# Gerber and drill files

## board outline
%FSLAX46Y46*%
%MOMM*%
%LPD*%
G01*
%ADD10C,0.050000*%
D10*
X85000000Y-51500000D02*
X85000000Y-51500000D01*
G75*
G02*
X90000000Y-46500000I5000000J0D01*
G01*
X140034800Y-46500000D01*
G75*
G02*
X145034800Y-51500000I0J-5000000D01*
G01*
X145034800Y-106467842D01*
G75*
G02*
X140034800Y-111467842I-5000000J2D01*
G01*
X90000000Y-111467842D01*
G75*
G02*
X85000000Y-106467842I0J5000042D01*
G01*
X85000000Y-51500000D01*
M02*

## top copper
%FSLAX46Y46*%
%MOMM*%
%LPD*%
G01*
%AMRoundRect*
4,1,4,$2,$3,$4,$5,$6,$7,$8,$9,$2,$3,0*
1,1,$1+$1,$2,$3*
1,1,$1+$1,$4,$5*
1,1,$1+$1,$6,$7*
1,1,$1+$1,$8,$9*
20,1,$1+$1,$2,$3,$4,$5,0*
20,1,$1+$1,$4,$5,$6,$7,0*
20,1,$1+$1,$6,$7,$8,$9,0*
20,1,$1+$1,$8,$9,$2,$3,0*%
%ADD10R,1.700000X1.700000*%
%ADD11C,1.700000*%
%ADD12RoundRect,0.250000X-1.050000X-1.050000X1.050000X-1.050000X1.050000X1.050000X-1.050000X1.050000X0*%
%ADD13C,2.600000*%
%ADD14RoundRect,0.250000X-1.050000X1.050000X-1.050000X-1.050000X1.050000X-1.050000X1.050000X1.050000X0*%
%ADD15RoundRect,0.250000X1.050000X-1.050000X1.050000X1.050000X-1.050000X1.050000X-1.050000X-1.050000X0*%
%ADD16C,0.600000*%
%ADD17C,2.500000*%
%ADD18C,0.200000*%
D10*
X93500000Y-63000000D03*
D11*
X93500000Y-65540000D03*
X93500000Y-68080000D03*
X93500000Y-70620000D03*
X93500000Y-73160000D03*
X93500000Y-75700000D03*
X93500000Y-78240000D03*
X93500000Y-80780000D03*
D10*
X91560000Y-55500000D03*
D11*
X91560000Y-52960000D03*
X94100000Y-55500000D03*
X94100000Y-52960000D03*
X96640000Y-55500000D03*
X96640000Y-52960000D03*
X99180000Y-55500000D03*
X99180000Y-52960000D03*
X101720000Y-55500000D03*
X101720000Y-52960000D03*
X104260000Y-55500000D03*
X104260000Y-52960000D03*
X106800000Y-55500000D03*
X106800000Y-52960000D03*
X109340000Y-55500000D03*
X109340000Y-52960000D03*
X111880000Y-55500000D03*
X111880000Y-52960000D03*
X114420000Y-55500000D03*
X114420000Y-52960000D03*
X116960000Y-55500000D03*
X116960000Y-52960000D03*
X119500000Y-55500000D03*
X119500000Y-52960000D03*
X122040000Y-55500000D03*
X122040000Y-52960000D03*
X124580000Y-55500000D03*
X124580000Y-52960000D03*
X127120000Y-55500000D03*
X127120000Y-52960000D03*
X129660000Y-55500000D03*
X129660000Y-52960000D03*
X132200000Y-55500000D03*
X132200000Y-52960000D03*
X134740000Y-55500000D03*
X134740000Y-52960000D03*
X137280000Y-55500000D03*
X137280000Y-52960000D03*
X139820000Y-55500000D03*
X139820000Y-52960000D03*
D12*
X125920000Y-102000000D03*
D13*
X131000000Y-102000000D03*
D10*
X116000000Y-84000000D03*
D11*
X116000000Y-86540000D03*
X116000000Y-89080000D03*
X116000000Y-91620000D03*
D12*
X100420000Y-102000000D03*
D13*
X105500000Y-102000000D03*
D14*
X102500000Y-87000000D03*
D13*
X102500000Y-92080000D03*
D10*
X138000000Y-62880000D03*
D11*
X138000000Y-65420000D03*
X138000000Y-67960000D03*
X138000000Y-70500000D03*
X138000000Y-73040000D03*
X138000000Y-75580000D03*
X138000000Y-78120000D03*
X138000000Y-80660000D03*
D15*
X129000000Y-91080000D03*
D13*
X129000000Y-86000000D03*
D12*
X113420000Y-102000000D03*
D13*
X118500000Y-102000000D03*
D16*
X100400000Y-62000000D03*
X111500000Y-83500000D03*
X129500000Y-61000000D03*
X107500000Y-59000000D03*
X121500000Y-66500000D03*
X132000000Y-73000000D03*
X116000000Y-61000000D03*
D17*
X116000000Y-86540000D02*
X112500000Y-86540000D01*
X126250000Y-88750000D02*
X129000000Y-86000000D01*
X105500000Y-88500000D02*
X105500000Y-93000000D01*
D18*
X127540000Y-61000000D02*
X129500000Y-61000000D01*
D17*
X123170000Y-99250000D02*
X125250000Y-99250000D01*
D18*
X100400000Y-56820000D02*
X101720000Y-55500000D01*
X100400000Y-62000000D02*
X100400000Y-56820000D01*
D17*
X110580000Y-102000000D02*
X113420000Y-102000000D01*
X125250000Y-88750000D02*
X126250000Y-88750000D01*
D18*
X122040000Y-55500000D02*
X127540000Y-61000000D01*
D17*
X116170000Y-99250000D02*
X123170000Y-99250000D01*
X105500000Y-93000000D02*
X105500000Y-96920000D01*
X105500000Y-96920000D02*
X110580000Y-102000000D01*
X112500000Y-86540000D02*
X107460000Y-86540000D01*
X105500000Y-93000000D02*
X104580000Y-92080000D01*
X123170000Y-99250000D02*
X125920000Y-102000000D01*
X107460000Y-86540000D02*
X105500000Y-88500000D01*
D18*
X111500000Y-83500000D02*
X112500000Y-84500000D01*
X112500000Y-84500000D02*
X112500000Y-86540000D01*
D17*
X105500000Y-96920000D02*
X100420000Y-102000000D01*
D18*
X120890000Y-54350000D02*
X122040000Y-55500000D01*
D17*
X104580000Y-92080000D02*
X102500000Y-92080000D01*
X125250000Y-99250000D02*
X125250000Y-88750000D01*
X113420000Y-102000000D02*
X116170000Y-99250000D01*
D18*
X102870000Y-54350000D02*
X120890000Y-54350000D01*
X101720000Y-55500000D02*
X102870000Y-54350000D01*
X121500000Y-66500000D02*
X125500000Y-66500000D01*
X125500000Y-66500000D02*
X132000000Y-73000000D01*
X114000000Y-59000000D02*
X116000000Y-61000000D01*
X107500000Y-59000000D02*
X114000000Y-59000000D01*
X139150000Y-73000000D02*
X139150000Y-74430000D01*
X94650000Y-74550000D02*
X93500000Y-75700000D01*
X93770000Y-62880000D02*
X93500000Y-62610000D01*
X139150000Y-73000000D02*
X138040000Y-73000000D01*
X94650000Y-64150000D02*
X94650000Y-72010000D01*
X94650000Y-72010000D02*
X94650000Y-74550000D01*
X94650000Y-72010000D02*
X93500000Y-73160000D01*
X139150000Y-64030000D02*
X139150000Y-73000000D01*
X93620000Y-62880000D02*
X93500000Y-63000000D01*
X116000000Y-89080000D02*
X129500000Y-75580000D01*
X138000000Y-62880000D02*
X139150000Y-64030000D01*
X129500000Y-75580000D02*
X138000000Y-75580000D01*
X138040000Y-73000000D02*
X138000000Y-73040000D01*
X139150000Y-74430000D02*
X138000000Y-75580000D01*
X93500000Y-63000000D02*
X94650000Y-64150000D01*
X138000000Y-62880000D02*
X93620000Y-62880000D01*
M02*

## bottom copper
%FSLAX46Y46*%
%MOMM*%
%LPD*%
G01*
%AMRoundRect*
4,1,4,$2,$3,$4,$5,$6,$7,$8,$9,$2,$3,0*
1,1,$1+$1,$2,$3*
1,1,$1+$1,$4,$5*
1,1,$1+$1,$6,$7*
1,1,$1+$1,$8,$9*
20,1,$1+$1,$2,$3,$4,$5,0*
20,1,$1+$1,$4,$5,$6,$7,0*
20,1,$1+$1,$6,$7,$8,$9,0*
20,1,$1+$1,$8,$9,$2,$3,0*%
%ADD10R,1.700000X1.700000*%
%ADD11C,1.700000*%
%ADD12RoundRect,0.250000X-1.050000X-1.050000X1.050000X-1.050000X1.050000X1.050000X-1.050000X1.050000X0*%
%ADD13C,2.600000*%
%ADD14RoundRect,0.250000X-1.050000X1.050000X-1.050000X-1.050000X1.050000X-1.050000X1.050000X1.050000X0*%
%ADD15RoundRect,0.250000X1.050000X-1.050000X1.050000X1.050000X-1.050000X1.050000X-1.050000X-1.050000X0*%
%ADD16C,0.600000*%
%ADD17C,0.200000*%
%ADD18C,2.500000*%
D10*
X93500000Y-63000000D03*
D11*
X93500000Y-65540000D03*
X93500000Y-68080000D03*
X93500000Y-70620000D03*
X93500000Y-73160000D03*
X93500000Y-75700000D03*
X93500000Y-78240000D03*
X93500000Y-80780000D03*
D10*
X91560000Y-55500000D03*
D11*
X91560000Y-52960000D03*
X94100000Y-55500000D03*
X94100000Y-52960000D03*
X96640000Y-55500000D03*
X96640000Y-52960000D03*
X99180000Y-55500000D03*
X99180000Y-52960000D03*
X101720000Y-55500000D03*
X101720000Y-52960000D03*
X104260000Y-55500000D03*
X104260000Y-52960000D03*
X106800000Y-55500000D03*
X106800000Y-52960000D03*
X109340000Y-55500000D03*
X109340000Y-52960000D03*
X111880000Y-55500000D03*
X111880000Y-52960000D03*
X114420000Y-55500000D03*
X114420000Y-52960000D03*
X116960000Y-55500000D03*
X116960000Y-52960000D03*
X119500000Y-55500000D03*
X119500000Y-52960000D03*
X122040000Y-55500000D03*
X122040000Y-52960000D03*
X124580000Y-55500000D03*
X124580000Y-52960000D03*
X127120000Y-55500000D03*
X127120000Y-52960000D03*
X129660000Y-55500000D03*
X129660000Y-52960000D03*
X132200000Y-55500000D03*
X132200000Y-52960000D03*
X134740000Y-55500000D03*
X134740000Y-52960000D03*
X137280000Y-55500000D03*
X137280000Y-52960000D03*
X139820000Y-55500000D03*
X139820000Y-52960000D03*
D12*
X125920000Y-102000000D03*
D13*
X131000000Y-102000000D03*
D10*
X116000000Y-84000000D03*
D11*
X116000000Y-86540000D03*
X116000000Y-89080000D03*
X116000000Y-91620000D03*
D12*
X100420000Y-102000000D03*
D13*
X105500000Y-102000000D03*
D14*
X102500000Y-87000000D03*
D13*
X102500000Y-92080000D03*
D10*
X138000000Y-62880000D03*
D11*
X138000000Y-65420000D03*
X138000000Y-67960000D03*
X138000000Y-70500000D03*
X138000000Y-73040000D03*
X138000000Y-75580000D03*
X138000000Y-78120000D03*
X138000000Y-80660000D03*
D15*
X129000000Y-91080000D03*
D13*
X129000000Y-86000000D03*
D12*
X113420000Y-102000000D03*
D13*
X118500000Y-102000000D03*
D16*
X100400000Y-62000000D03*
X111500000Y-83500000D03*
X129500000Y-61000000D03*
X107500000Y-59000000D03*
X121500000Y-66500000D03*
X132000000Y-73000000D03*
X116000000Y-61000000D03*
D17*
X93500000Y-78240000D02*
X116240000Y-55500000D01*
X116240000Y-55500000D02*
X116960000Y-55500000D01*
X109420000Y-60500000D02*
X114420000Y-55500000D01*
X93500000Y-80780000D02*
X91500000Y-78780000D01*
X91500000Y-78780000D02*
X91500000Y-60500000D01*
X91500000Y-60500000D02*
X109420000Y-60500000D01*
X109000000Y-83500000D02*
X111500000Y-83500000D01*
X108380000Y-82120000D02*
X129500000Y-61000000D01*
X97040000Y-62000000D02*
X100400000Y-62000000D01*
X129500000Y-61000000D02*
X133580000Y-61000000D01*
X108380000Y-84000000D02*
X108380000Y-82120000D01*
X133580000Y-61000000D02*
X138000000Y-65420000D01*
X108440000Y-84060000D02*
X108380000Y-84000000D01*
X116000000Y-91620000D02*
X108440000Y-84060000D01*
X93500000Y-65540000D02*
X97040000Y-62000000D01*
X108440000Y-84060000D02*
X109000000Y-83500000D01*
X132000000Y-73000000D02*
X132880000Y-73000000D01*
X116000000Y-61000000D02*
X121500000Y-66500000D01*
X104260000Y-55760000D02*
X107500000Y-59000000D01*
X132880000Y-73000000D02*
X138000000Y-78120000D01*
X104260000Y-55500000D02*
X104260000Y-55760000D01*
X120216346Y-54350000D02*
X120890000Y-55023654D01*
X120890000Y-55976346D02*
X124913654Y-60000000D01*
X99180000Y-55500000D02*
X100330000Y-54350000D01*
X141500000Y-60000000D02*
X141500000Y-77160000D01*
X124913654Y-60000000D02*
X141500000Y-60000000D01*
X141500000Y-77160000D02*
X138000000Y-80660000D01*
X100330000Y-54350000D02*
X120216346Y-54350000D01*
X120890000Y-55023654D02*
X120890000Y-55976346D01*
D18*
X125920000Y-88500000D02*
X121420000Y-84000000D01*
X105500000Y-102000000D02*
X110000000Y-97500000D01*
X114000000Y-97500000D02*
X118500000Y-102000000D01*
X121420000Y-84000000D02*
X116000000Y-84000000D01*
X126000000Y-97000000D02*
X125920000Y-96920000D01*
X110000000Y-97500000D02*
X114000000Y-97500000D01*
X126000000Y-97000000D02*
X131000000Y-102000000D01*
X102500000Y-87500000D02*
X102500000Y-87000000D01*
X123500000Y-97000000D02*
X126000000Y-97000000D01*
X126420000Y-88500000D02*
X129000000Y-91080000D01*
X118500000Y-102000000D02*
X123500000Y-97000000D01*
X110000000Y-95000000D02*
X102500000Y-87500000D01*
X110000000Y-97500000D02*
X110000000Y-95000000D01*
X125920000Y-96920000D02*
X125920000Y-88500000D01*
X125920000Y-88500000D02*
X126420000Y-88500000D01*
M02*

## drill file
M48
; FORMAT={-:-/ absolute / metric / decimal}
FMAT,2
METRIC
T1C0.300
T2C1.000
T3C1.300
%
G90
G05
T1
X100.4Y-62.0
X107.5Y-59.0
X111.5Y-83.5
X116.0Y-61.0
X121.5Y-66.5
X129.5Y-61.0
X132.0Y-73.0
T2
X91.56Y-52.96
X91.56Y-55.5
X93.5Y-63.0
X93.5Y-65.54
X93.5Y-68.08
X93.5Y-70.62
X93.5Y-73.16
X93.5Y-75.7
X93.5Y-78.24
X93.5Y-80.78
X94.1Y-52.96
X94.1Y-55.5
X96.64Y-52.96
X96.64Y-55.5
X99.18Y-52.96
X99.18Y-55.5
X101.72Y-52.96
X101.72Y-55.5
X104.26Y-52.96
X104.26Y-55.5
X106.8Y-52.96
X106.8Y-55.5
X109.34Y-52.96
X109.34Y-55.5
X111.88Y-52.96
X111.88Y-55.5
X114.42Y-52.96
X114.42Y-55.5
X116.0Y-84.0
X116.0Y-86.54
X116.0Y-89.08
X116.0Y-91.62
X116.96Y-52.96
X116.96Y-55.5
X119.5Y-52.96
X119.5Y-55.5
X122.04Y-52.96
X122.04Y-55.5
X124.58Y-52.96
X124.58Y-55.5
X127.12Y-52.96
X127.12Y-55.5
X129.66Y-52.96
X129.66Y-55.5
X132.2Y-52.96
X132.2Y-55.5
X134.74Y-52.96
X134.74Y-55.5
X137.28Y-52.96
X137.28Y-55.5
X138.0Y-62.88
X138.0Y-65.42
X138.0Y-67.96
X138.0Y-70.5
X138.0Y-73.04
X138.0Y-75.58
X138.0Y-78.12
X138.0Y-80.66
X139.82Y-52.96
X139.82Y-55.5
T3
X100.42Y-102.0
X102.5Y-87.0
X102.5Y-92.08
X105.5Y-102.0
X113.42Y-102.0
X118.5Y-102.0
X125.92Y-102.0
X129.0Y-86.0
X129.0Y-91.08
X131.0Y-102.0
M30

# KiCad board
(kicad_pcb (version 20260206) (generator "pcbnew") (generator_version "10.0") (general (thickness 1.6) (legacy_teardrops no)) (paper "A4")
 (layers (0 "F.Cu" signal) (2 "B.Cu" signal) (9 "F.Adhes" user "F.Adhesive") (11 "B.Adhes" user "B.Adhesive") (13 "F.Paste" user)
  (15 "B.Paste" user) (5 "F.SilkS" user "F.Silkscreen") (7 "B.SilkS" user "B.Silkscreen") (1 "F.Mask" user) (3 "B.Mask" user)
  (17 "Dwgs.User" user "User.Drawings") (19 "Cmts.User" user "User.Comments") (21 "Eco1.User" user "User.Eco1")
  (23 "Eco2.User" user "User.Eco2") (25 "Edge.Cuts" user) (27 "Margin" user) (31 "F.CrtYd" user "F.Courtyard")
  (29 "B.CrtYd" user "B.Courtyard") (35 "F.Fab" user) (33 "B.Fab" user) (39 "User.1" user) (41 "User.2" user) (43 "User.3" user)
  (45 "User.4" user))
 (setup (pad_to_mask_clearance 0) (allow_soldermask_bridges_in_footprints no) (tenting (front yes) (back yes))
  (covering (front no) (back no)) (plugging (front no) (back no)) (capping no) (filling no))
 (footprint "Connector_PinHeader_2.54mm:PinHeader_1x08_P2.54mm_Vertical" (layer "F.Cu") (at 93.5 63)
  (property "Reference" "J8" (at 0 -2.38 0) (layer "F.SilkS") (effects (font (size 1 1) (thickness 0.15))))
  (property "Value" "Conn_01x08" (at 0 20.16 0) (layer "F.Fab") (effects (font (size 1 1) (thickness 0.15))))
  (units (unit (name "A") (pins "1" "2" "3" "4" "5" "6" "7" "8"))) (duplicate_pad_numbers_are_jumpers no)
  (pad "1" thru_hole rect (at 0 0) (size 1.7 1.7) (drill 1) (layers "*.Cu" "*.Mask") (remove_unused_layers no) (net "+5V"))
  (pad "2" thru_hole circle (at 0 2.54) (size 1.7 1.7) (drill 1) (layers "*.Cu" "*.Mask") (remove_unused_layers no) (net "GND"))
  (pad "3" thru_hole circle (at 0 5.08) (size 1.7 1.7) (drill 1) (layers "*.Cu" "*.Mask") (remove_unused_layers no)
   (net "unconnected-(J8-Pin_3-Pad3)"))
  (pad "4" thru_hole circle (at 0 7.62) (size 1.7 1.7) (drill 1) (layers "*.Cu" "*.Mask") (remove_unused_layers no)
   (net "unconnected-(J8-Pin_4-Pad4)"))
  (pad "5" thru_hole circle (at 0 10.16) (size 1.7 1.7) (drill 1) (layers "*.Cu" "*.Mask") (remove_unused_layers no) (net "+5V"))
  (pad "6" thru_hole circle (at 0 12.7) (size 1.7 1.7) (drill 1) (layers "*.Cu" "*.Mask") (remove_unused_layers no) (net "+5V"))
  (pad "7" thru_hole circle (at 0 15.24) (size 1.7 1.7) (drill 1) (layers "*.Cu" "*.Mask") (remove_unused_layers no) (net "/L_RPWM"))
  (pad "8" thru_hole circle (at 0 17.78) (size 1.7 1.7) (drill 1) (layers "*.Cu" "*.Mask") (remove_unused_layers no) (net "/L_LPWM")))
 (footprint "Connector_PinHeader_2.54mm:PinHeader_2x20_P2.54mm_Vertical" (layer "F.Cu") (at 91.56 55.5 90)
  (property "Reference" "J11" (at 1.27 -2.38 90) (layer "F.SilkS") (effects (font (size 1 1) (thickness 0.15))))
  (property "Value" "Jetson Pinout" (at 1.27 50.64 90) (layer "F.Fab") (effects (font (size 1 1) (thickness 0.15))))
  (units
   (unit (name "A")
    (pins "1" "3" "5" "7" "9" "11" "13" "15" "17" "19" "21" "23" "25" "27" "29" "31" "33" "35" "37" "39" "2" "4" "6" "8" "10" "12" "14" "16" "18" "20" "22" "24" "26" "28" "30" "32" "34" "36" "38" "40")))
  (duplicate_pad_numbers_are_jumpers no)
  (pad "1" thru_hole rect (at 0 0 90) (size 1.7 1.7) (drill 1) (layers "*.Cu" "*.Mask") (remove_unused_layers no) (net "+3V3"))
  (pad "2" thru_hole circle (at 2.54 0 90) (size 1.7 1.7) (drill 1) (layers "*.Cu" "*.Mask") (remove_unused_layers no)
   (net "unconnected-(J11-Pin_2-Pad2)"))
  (pad "3" thru_hole circle (at 0 2.54 90) (size 1.7 1.7) (drill 1) (layers "*.Cu" "*.Mask") (remove_unused_layers no)
   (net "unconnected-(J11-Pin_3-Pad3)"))
  (pad "4" thru_hole circle (at 2.54 2.54 90) (size 1.7 1.7) (drill 1) (layers "*.Cu" "*.Mask") (remove_unused_layers no)
   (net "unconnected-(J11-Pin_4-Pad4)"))
  (pad "5" thru_hole circle (at 0 5.08 90) (size 1.7 1.7) (drill 1) (layers "*.Cu" "*.Mask") (remove_unused_layers no)
   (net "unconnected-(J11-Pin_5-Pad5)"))
  (pad "6" thru_hole circle (at 2.54 5.08 90) (size 1.7 1.7) (drill 1) (layers "*.Cu" "*.Mask") (remove_unused_layers no)
   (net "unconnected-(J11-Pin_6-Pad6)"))
  (pad "7" thru_hole circle (at 0 7.62 90) (size 1.7 1.7) (drill 1) (layers "*.Cu" "*.Mask") (remove_unused_layers no) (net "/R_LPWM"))
  (pad "8" thru_hole circle (at 2.54 7.62 90) (size 1.7 1.7) (drill 1) (layers "*.Cu" "*.Mask") (remove_unused_layers no)
   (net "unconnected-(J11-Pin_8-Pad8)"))
  (pad "9" thru_hole circle (at 0 10.16 90) (size 1.7 1.7) (drill 1) (layers "*.Cu" "*.Mask") (remove_unused_layers no) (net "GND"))
  (pad "10" thru_hole circle (at 2.54 10.16 90) (size 1.7 1.7) (drill 1) (layers "*.Cu" "*.Mask") (remove_unused_layers no)
   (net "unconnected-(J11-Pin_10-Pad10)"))
  (pad "11" thru_hole circle (at 0 12.7 90) (size 1.7 1.7) (drill 1) (layers "*.Cu" "*.Mask") (remove_unused_layers no) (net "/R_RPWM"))
  (pad "12" thru_hole circle (at 2.54 12.7 90) (size 1.7 1.7) (drill 1) (layers "*.Cu" "*.Mask") (remove_unused_layers no)
   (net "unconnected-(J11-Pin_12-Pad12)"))
  (pad "13" thru_hole circle (at 0 15.24 90) (size 1.7 1.7) (drill 1) (layers "*.Cu" "*.Mask") (remove_unused_layers no)
   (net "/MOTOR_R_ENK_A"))
  (pad "14" thru_hole circle (at 2.54 15.24 90) (size 1.7 1.7) (drill 1) (layers "*.Cu" "*.Mask") (remove_unused_layers no)
   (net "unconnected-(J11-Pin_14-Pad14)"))
  (pad "15" thru_hole circle (at 0 17.78 90) (size 1.7 1.7) (drill 1) (layers "*.Cu" "*.Mask") (remove_unused_layers no)
   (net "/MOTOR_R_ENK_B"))
  (pad "16" thru_hole circle (at 2.54 17.78 90) (size 1.7 1.7) (drill 1) (layers "*.Cu" "*.Mask") (remove_unused_layers no)
   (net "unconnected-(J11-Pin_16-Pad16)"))
  (pad "17" thru_hole circle (at 0 20.32 90) (size 1.7 1.7) (drill 1) (layers "*.Cu" "*.Mask") (remove_unused_layers no)
   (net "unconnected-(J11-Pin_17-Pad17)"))
  (pad "18" thru_hole circle (at 2.54 20.32 90) (size 1.7 1.7) (drill 1) (layers "*.Cu" "*.Mask") (remove_unused_layers no)
   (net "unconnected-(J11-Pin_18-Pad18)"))
  (pad "19" thru_hole circle (at 0 22.86 90) (size 1.7 1.7) (drill 1) (layers "*.Cu" "*.Mask") (remove_unused_layers no) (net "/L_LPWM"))
  (pad "20" thru_hole circle (at 2.54 22.86 90) (size 1.7 1.7) (drill 1) (layers "*.Cu" "*.Mask") (remove_unused_layers no)
   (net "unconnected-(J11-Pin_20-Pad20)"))
  (pad "21" thru_hole circle (at 0 25.4 90) (size 1.7 1.7) (drill 1) (layers "*.Cu" "*.Mask") (remove_unused_layers no) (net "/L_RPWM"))
  (pad "22" thru_hole circle (at 2.54 25.4 90) (size 1.7 1.7) (drill 1) (layers "*.Cu" "*.Mask") (remove_unused_layers no)
   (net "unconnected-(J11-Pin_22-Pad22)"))
  (pad "23" thru_hole circle (at 0 27.94 90) (size 1.7 1.7) (drill 1) (layers "*.Cu" "*.Mask") (remove_unused_layers no)
   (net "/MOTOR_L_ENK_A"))
  (pad "24" thru_hole circle (at 2.54 27.94 90) (size 1.7 1.7) (drill 1) (layers "*.Cu" "*.Mask") (remove_unused_layers no)
   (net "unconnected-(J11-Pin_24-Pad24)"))
  (pad "25" thru_hole circle (at 0 30.48 90) (size 1.7 1.7) (drill 1) (layers "*.Cu" "*.Mask") (remove_unused_layers no) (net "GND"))
  (pad "26" thru_hole circle (at 2.54 30.48 90) (size 1.7 1.7) (drill 1) (layers "*.Cu" "*.Mask") (remove_unused_layers no)
   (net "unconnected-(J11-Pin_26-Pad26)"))
  (pad "27" thru_hole circle (at 0 33.02 90) (size 1.7 1.7) (drill 1) (layers "*.Cu" "*.Mask") (remove_unused_layers no)
   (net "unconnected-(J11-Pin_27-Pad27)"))
  (pad "28" thru_hole circle (at 2.54 33.02 90) (size 1.7 1.7) (drill 1) (layers "*.Cu" "*.Mask") (remove_unused_layers no)
   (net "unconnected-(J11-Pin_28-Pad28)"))
  (pad "29" thru_hole circle (at 0 35.56 90) (size 1.7 1.7) (drill 1) (layers "*.Cu" "*.Mask") (remove_unused_layers no)
   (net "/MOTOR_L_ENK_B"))
  (pad "30" thru_hole circle (at 2.54 35.56 90) (size 1.7 1.7) (drill 1) (layers "*.Cu" "*.Mask") (remove_unused_layers no)
   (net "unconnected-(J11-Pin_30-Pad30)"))
  (pad "31" thru_hole circle (at 0 38.1 90) (size 1.7 1.7) (drill 1) (layers "*.Cu" "*.Mask") (remove_unused_layers no)
   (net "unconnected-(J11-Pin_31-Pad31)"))
  (pad "32" thru_hole circle (at 2.54 38.1 90) (size 1.7 1.7) (drill 1) (layers "*.Cu" "*.Mask") (remove_unused_layers no)
   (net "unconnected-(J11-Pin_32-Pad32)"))
  (pad "33" thru_hole circle (at 0 40.64 90) (size 1.7 1.7) (drill 1) (layers "*.Cu" "*.Mask") (remove_unused_layers no)
   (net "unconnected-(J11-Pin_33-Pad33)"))
  (pad "34" thru_hole circle (at 2.54 40.64 90) (size 1.7 1.7) (drill 1) (layers "*.Cu" "*.Mask") (remove_unused_layers no)
   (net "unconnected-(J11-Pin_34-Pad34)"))
  (pad "35" thru_hole circle (at 0 43.18 90) (size 1.7 1.7) (drill 1) (layers "*.Cu" "*.Mask") (remove_unused_layers no)
   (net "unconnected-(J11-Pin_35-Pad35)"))
  (pad "36" thru_hole circle (at 2.54 43.18 90) (size 1.7 1.7) (drill 1) (layers "*.Cu" "*.Mask") (remove_unused_layers no)
   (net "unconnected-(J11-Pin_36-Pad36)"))
  (pad "37" thru_hole circle (at 0 45.72 90) (size 1.7 1.7) (drill 1) (layers "*.Cu" "*.Mask") (remove_unused_layers no)
   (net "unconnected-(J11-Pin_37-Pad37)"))
  (pad "38" thru_hole circle (at 2.54 45.72 90) (size 1.7 1.7) (drill 1) (layers "*.Cu" "*.Mask") (remove_unused_layers no)
   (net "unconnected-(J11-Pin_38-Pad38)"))
  (pad "39" thru_hole circle (at 0 48.26 90) (size 1.7 1.7) (drill 1) (layers "*.Cu" "*.Mask") (remove_unused_layers no)
   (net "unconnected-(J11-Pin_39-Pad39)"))
  (pad "40" thru_hole circle (at 2.54 48.26 90) (size 1.7 1.7) (drill 1) (layers "*.Cu" "*.Mask") (remove_unused_layers no)
   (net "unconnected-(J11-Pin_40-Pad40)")))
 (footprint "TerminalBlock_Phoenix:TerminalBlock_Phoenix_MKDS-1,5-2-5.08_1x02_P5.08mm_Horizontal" (layer "F.Cu") (at 125.92 102)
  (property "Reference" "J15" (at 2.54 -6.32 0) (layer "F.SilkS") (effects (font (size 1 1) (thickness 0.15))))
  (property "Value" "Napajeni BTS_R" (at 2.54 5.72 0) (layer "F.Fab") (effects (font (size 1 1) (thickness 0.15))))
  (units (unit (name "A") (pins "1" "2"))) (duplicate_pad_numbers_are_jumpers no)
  (pad "1" thru_hole roundrect (at 0 0) (size 2.6 2.6) (drill 1.3) (layers "*.Cu" "*.Mask") (remove_unused_layers no)
   (roundrect_rratio 0.096154) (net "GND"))
  (pad "2" thru_hole circle (at 5.08 0) (size 2.6 2.6) (drill 1.3) (layers "*.Cu" "*.Mask") (remove_unused_layers no) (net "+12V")))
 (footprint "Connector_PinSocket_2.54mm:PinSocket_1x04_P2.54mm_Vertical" (layer "F.Cu") (at 116 84)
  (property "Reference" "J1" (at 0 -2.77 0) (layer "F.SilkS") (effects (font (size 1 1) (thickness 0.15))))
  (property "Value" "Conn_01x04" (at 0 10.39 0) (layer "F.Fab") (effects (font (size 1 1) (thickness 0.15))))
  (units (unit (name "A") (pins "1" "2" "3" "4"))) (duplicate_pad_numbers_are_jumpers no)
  (pad "1" thru_hole rect (at 0 0) (size 1.7 1.7) (drill 1) (layers "*.Cu" "*.Mask") (remove_unused_layers no) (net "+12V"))
  (pad "2" thru_hole circle (at 0 2.54) (size 1.7 1.7) (drill 1) (layers "*.Cu" "*.Mask") (remove_unused_layers no) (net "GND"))
  (pad "3" thru_hole circle (at 0 5.08) (size 1.7 1.7) (drill 1) (layers "*.Cu" "*.Mask") (remove_unused_layers no) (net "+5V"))
  (pad "4" thru_hole circle (at 0 7.62) (size 1.7 1.7) (drill 1) (layers "*.Cu" "*.Mask") (remove_unused_layers no) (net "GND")))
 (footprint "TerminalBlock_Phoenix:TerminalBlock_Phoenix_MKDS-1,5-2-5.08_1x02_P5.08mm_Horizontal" (layer "F.Cu") (at 100.42 102)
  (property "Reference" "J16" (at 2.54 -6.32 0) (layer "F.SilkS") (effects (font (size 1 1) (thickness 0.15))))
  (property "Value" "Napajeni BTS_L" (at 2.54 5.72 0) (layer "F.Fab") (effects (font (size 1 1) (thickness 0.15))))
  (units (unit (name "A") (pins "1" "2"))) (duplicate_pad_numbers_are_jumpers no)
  (pad "1" thru_hole roundrect (at 0 0) (size 2.6 2.6) (drill 1.3) (layers "*.Cu" "*.Mask") (remove_unused_layers no)
   (roundrect_rratio 0.096154) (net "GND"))
  (pad "2" thru_hole circle (at 5.08 0) (size 2.6 2.6) (drill 1.3) (layers "*.Cu" "*.Mask") (remove_unused_layers no) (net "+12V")))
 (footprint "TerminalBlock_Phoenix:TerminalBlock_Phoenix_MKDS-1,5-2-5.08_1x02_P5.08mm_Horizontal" (layer "F.Cu") (at 102.5 87 -90)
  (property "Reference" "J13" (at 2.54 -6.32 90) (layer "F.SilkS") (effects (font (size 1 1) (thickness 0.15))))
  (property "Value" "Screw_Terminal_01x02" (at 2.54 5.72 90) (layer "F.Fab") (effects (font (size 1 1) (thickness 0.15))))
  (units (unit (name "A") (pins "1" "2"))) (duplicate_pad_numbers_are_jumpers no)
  (pad "1" thru_hole roundrect (at 0 0 270) (size 2.6 2.6) (drill 1.3) (layers "*.Cu" "*.Mask") (remove_unused_layers no)
   (roundrect_rratio 0.096154) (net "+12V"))
  (pad "2" thru_hole circle (at 5.08 0 270) (size 2.6 2.6) (drill 1.3) (layers "*.Cu" "*.Mask") (remove_unused_layers no) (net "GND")))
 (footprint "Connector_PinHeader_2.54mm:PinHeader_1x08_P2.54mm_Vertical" (layer "F.Cu") (at 138 62.88)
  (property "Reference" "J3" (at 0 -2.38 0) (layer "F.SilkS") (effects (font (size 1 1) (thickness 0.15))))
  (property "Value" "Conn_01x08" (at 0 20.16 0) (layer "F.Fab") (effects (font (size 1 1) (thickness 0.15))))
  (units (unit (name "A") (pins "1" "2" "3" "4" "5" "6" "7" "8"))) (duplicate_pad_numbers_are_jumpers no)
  (pad "1" thru_hole rect (at 0 0) (size 1.7 1.7) (drill 1) (layers "*.Cu" "*.Mask") (remove_unused_layers no) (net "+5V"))
  (pad "2" thru_hole circle (at 0 2.54) (size 1.7 1.7) (drill 1) (layers "*.Cu" "*.Mask") (remove_unused_layers no) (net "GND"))
  (pad "3" thru_hole circle (at 0 5.08) (size 1.7 1.7) (drill 1) (layers "*.Cu" "*.Mask") (remove_unused_layers no)
   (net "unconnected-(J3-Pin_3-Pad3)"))
  (pad "4" thru_hole circle (at 0 7.62) (size 1.7 1.7) (drill 1) (layers "*.Cu" "*.Mask") (remove_unused_layers no)
   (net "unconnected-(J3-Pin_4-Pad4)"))
  (pad "5" thru_hole circle (at 0 10.16) (size 1.7 1.7) (drill 1) (layers "*.Cu" "*.Mask") (remove_unused_layers no) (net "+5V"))
  (pad "6" thru_hole circle (at 0 12.7) (size 1.7 1.7) (drill 1) (layers "*.Cu" "*.Mask") (remove_unused_layers no) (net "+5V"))
  (pad "7" thru_hole circle (at 0 15.24) (size 1.7 1.7) (drill 1) (layers "*.Cu" "*.Mask") (remove_unused_layers no) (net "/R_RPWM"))
  (pad "8" thru_hole circle (at 0 17.78) (size 1.7 1.7) (drill 1) (layers "*.Cu" "*.Mask") (remove_unused_layers no) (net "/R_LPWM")))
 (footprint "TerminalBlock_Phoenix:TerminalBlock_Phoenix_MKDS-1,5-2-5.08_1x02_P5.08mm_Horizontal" (layer "F.Cu") (at 129 91.08 90)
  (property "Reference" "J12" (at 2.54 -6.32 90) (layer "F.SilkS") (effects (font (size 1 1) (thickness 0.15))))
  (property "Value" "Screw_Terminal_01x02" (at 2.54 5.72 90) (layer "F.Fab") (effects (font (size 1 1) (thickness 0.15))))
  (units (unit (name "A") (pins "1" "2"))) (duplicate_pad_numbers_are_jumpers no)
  (pad "1" thru_hole roundrect (at 0 0 90) (size 2.6 2.6) (drill 1.3) (layers "*.Cu" "*.Mask") (remove_unused_layers no)
   (roundrect_rratio 0.096154) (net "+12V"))
  (pad "2" thru_hole circle (at 5.08 0 90) (size 2.6 2.6) (drill 1.3) (layers "*.Cu" "*.Mask") (remove_unused_layers no) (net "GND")))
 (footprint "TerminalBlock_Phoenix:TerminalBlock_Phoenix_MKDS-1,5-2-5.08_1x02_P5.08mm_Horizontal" (layer "F.Cu") (at 113.42 102)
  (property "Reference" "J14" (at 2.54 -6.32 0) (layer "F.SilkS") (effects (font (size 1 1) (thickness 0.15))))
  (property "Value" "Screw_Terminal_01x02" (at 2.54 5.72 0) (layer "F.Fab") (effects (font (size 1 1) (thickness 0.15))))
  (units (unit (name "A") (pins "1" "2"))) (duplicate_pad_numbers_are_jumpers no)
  (pad "1" thru_hole roundrect (at 0 0) (size 2.6 2.6) (drill 1.3) (layers "*.Cu" "*.Mask") (remove_unused_layers no)
   (roundrect_rratio 0.096154) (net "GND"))
  (pad "2" thru_hole circle (at 5.08 0) (size 2.6 2.6) (drill 1.3) (layers "*.Cu" "*.Mask") (remove_unused_layers no) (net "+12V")))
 (gr_rect (start 85 46.5) (end 145.0348 111.467842) (radius 5) (stroke (width 0.05) (type solid)) (fill no) (layer "Edge.Cuts"))
 (segment (start 93.5 78.24) (end 116.24 55.5) (width 0.2) (layer "B.Cu") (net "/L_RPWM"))
 (segment (start 116.24 55.5) (end 116.96 55.5) (width 0.2) (layer "B.Cu") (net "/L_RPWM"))
 (segment (start 109.42 60.5) (end 114.42 55.5) (width 0.2) (layer "B.Cu") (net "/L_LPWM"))
 (segment (start 93.5 80.78) (end 91.5 78.78) (width 0.2) (layer "B.Cu") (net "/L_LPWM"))
 (segment (start 91.5 78.78) (end 91.5 60.5) (width 0.2) (layer "B.Cu") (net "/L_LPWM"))
 (segment (start 91.5 60.5) (end 109.42 60.5) (width 0.2) (layer "B.Cu") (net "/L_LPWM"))
 (segment (start 116 86.54) (end 112.5 86.54) (width 2.5) (layer "F.Cu") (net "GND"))
 (segment (start 126.25 88.75) (end 129 86) (width 2.5) (layer "F.Cu") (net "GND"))
 (segment (start 105.5 88.5) (end 105.5 93) (width 2.5) (layer "F.Cu") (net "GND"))
 (segment (start 127.54 61) (end 129.5 61) (width 0.2) (layer "F.Cu") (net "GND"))
 (segment (start 123.17 99.25) (end 125.25 99.25) (width 2.5) (layer "F.Cu") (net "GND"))
 (segment (start 100.4 56.82) (end 101.72 55.5) (width 0.2) (layer "F.Cu") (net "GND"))
 (segment (start 100.4 62) (end 100.4 56.82) (width 0.2) (layer "F.Cu") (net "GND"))
 (segment (start 110.58 102) (end 113.42 102) (width 2.5) (layer "F.Cu") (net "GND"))
 (segment (start 125.25 88.75) (end 126.25 88.75) (width 2.5) (layer "F.Cu") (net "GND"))
 (segment (start 122.04 55.5) (end 127.54 61) (width 0.2) (layer "F.Cu") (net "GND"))
 (segment (start 116.17 99.25) (end 123.17 99.25) (width 2.5) (layer "F.Cu") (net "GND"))
 (segment (start 105.5 93) (end 105.5 96.92) (width 2.5) (layer "F.Cu") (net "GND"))
 (segment (start 105.5 96.92) (end 110.58 102) (width 2.5) (layer "F.Cu") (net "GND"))
 (segment (start 112.5 86.54) (end 107.46 86.54) (width 2.5) (layer "F.Cu") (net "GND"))
 (segment (start 105.5 93) (end 104.58 92.08) (width 2.5) (layer "F.Cu") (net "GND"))
 (segment (start 123.17 99.25) (end 125.92 102) (width 2.5) (layer "F.Cu") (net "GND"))
 (segment (start 107.46 86.54) (end 105.5 88.5) (width 2.5) (layer "F.Cu") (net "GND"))
 (segment (start 111.5 83.5) (end 112.5 84.5) (width 0.2) (layer "F.Cu") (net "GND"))
 (segment (start 112.5 84.5) (end 112.5 86.54) (width 0.2) (layer "F.Cu") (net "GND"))
 (segment (start 105.5 96.92) (end 100.42 102) (width 2.5) (layer "F.Cu") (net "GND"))
 (segment (start 120.89 54.35) (end 122.04 55.5) (width 0.2) (layer "F.Cu") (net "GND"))
 (segment (start 104.58 92.08) (end 102.5 92.08) (width 2.5) (layer "F.Cu") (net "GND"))
 (segment (start 125.25 99.25) (end 125.25 88.75) (width 2.5) (layer "F.Cu") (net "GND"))
 (segment (start 113.42 102) (end 116.17 99.25) (width 2.5) (layer "F.Cu") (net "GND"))
 (segment (start 102.87 54.35) (end 120.89 54.35) (width 0.2) (layer "F.Cu") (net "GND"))
 (segment (start 101.72 55.5) (end 102.87 54.35) (width 0.2) (layer "F.Cu") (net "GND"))
 (via (at 100.4 62) (size 0.6) (drill 0.3) (layers "F.Cu" "B.Cu") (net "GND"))
 (via (at 111.5 83.5) (size 0.6) (drill 0.3) (layers "F.Cu" "B.Cu") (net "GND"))
 (via (at 129.5 61) (size 0.6) (drill 0.3) (layers "F.Cu" "B.Cu") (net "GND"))
 (segment (start 109 83.5) (end 111.5 83.5) (width 0.2) (layer "B.Cu") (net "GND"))
 (segment (start 108.38 82.12) (end 129.5 61) (width 0.2) (layer "B.Cu") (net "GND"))
 (segment (start 97.04 62) (end 100.4 62) (width 0.2) (layer "B.Cu") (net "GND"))
 (segment (start 129.5 61) (end 133.58 61) (width 0.2) (layer "B.Cu") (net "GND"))
 (segment (start 108.38 84) (end 108.38 82.12) (width 0.2) (layer "B.Cu") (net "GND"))
 (segment (start 133.58 61) (end 138 65.42) (width 0.2) (layer "B.Cu") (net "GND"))
 (segment (start 108.44 84.06) (end 108.38 84) (width 0.2) (layer "B.Cu") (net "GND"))
 (segment (start 116 91.62) (end 108.44 84.06) (width 0.2) (layer "B.Cu") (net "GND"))
 (segment (start 93.5 65.54) (end 97.04 62) (width 0.2) (layer "B.Cu") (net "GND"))
 (segment (start 108.44 84.06) (end 109 83.5) (width 0.2) (layer "B.Cu") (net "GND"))
 (segment (start 121.5 66.5) (end 125.5 66.5) (width 0.2) (layer "F.Cu") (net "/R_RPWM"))
 (segment (start 125.5 66.5) (end 132 73) (width 0.2) (layer "F.Cu") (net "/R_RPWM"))
 (segment (start 114 59) (end 116 61) (width 0.2) (layer "F.Cu") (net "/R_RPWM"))
 (segment (start 107.5 59) (end 114 59) (width 0.2) (layer "F.Cu") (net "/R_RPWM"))
 (via (at 107.5 59) (size 0.6) (drill 0.3) (layers "F.Cu" "B.Cu") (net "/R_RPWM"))
 (via (at 121.5 66.5) (size 0.6) (drill 0.3) (layers "F.Cu" "B.Cu") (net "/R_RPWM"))
 (via (at 132 73) (size 0.6) (drill 0.3) (layers "F.Cu" "B.Cu") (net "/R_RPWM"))
 (via (at 116 61) (size 0.6) (drill 0.3) (layers "F.Cu" "B.Cu") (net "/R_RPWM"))
 (segment (start 132 73) (end 132.88 73) (width 0.2) (layer "B.Cu") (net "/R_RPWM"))
 (segment (start 116 61) (end 121.5 66.5) (width 0.2) (layer "B.Cu") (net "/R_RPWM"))
 (segment (start 104.26 55.76) (end 107.5 59) (width 0.2) (layer "B.Cu") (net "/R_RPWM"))
 (segment (start 132.88 73) (end 138 78.12) (width 0.2) (layer "B.Cu") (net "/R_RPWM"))
 (segment (start 104.26 55.5) (end 104.26 55.76) (width 0.2) (layer "B.Cu") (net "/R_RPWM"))
 (segment (start 120.216346 54.35) (end 120.89 55.023654) (width 0.2) (layer "B.Cu") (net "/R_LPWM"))
 (segment (start 120.89 55.976346) (end 124.913654 60) (width 0.2) (layer "B.Cu") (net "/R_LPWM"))
 (segment (start 99.18 55.5) (end 100.33 54.35) (width 0.2) (layer "B.Cu") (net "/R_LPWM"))
 (segment (start 141.5 60) (end 141.5 77.16) (width 0.2) (layer "B.Cu") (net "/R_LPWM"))
 (segment (start 124.913654 60) (end 141.5 60) (width 0.2) (layer "B.Cu") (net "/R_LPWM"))
 (segment (start 141.5 77.16) (end 138 80.66) (width 0.2) (layer "B.Cu") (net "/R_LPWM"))
 (segment (start 100.33 54.35) (end 120.216346 54.35) (width 0.2) (layer "B.Cu") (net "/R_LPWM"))
 (segment (start 120.89 55.023654) (end 120.89 55.976346) (width 0.2) (layer "B.Cu") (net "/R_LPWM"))
 (segment (start 125.92 88.5) (end 121.42 84) (width 2.5) (layer "B.Cu") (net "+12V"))
 (segment (start 105.5 102) (end 110 97.5) (width 2.5) (layer "B.Cu") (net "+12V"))
 (segment (start 114 97.5) (end 118.5 102) (width 2.5) (layer "B.Cu") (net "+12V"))
 (segment (start 121.42 84) (end 116 84) (width 2.5) (layer "B.Cu") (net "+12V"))
 (segment (start 126 97) (end 125.92 96.92) (width 2.5) (layer "B.Cu") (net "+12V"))
 (segment (start 110 97.5) (end 114 97.5) (width 2.5) (layer "B.Cu") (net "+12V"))
 (segment (start 126 97) (end 131 102) (width 2.5) (layer "B.Cu") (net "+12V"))
 (segment (start 102.5 87.5) (end 102.5 87) (width 2.5) (layer "B.Cu") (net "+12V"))
 (segment (start 123.5 97) (end 126 97) (width 2.5) (layer "B.Cu") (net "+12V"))
 (segment (start 126.42 88.5) (end 129 91.08) (width 2.5) (layer "B.Cu") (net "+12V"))
 (segment (start 118.5 102) (end 123.5 97) (width 2.5) (layer "B.Cu") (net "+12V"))
 (segment (start 110 95) (end 102.5 87.5) (width 2.5) (layer "B.Cu") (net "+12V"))
 (segment (start 110 97.5) (end 110 95) (width 2.5) (layer "B.Cu") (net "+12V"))
 (segment (start 125.92 96.92) (end 125.92 88.5) (width 2.5) (layer "B.Cu") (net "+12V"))
 (segment (start 125.92 88.5) (end 126.42 88.5) (width 2.5) (layer "B.Cu") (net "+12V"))
 (segment (start 139.15 73) (end 139.15 74.43) (width 0.2) (layer "F.Cu") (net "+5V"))
 (segment (start 94.65 74.55) (end 93.5 75.7) (width 0.2) (layer "F.Cu") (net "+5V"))
 (segment (start 93.77 62.88) (end 93.5 62.61) (width 0.2) (layer "F.Cu") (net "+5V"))
 (segment (start 139.15 73) (end 138.04 73) (width 0.2) (layer "F.Cu") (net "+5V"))
 (segment (start 94.65 64.15) (end 94.65 72.01) (width 0.2) (layer "F.Cu") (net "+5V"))
 (segment (start 94.65 72.01) (end 94.65 74.55) (width 0.2) (layer "F.Cu") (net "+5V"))
 (segment (start 94.65 72.01) (end 93.5 73.16) (width 0.2) (layer "F.Cu") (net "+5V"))
 (segment (start 139.15 64.03) (end 139.15 73) (width 0.2) (layer "F.Cu") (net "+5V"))
 (segment (start 93.62 62.88) (end 93.5 63) (width 0.2) (layer "F.Cu") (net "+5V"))
 (segment (start 116 89.08) (end 129.5 75.58) (width 0.2) (layer "F.Cu") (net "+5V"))
 (segment (start 138 62.88) (end 139.15 64.03) (width 0.2) (layer "F.Cu") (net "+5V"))
 (segment (start 129.5 75.58) (end 138 75.58) (width 0.2) (layer "F.Cu") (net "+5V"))
 (segment (start 138.04 73) (end 138 73.04) (width 0.2) (layer "F.Cu") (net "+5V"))
 (segment (start 139.15 74.43) (end 138 75.58) (width 0.2) (layer "F.Cu") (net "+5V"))
 (segment (start 93.5 63) (end 94.65 64.15) (width 0.2) (layer "F.Cu") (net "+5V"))
 (segment (start 138 62.88) (end 93.62 62.88) (width 0.2) (layer "F.Cu") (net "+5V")))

